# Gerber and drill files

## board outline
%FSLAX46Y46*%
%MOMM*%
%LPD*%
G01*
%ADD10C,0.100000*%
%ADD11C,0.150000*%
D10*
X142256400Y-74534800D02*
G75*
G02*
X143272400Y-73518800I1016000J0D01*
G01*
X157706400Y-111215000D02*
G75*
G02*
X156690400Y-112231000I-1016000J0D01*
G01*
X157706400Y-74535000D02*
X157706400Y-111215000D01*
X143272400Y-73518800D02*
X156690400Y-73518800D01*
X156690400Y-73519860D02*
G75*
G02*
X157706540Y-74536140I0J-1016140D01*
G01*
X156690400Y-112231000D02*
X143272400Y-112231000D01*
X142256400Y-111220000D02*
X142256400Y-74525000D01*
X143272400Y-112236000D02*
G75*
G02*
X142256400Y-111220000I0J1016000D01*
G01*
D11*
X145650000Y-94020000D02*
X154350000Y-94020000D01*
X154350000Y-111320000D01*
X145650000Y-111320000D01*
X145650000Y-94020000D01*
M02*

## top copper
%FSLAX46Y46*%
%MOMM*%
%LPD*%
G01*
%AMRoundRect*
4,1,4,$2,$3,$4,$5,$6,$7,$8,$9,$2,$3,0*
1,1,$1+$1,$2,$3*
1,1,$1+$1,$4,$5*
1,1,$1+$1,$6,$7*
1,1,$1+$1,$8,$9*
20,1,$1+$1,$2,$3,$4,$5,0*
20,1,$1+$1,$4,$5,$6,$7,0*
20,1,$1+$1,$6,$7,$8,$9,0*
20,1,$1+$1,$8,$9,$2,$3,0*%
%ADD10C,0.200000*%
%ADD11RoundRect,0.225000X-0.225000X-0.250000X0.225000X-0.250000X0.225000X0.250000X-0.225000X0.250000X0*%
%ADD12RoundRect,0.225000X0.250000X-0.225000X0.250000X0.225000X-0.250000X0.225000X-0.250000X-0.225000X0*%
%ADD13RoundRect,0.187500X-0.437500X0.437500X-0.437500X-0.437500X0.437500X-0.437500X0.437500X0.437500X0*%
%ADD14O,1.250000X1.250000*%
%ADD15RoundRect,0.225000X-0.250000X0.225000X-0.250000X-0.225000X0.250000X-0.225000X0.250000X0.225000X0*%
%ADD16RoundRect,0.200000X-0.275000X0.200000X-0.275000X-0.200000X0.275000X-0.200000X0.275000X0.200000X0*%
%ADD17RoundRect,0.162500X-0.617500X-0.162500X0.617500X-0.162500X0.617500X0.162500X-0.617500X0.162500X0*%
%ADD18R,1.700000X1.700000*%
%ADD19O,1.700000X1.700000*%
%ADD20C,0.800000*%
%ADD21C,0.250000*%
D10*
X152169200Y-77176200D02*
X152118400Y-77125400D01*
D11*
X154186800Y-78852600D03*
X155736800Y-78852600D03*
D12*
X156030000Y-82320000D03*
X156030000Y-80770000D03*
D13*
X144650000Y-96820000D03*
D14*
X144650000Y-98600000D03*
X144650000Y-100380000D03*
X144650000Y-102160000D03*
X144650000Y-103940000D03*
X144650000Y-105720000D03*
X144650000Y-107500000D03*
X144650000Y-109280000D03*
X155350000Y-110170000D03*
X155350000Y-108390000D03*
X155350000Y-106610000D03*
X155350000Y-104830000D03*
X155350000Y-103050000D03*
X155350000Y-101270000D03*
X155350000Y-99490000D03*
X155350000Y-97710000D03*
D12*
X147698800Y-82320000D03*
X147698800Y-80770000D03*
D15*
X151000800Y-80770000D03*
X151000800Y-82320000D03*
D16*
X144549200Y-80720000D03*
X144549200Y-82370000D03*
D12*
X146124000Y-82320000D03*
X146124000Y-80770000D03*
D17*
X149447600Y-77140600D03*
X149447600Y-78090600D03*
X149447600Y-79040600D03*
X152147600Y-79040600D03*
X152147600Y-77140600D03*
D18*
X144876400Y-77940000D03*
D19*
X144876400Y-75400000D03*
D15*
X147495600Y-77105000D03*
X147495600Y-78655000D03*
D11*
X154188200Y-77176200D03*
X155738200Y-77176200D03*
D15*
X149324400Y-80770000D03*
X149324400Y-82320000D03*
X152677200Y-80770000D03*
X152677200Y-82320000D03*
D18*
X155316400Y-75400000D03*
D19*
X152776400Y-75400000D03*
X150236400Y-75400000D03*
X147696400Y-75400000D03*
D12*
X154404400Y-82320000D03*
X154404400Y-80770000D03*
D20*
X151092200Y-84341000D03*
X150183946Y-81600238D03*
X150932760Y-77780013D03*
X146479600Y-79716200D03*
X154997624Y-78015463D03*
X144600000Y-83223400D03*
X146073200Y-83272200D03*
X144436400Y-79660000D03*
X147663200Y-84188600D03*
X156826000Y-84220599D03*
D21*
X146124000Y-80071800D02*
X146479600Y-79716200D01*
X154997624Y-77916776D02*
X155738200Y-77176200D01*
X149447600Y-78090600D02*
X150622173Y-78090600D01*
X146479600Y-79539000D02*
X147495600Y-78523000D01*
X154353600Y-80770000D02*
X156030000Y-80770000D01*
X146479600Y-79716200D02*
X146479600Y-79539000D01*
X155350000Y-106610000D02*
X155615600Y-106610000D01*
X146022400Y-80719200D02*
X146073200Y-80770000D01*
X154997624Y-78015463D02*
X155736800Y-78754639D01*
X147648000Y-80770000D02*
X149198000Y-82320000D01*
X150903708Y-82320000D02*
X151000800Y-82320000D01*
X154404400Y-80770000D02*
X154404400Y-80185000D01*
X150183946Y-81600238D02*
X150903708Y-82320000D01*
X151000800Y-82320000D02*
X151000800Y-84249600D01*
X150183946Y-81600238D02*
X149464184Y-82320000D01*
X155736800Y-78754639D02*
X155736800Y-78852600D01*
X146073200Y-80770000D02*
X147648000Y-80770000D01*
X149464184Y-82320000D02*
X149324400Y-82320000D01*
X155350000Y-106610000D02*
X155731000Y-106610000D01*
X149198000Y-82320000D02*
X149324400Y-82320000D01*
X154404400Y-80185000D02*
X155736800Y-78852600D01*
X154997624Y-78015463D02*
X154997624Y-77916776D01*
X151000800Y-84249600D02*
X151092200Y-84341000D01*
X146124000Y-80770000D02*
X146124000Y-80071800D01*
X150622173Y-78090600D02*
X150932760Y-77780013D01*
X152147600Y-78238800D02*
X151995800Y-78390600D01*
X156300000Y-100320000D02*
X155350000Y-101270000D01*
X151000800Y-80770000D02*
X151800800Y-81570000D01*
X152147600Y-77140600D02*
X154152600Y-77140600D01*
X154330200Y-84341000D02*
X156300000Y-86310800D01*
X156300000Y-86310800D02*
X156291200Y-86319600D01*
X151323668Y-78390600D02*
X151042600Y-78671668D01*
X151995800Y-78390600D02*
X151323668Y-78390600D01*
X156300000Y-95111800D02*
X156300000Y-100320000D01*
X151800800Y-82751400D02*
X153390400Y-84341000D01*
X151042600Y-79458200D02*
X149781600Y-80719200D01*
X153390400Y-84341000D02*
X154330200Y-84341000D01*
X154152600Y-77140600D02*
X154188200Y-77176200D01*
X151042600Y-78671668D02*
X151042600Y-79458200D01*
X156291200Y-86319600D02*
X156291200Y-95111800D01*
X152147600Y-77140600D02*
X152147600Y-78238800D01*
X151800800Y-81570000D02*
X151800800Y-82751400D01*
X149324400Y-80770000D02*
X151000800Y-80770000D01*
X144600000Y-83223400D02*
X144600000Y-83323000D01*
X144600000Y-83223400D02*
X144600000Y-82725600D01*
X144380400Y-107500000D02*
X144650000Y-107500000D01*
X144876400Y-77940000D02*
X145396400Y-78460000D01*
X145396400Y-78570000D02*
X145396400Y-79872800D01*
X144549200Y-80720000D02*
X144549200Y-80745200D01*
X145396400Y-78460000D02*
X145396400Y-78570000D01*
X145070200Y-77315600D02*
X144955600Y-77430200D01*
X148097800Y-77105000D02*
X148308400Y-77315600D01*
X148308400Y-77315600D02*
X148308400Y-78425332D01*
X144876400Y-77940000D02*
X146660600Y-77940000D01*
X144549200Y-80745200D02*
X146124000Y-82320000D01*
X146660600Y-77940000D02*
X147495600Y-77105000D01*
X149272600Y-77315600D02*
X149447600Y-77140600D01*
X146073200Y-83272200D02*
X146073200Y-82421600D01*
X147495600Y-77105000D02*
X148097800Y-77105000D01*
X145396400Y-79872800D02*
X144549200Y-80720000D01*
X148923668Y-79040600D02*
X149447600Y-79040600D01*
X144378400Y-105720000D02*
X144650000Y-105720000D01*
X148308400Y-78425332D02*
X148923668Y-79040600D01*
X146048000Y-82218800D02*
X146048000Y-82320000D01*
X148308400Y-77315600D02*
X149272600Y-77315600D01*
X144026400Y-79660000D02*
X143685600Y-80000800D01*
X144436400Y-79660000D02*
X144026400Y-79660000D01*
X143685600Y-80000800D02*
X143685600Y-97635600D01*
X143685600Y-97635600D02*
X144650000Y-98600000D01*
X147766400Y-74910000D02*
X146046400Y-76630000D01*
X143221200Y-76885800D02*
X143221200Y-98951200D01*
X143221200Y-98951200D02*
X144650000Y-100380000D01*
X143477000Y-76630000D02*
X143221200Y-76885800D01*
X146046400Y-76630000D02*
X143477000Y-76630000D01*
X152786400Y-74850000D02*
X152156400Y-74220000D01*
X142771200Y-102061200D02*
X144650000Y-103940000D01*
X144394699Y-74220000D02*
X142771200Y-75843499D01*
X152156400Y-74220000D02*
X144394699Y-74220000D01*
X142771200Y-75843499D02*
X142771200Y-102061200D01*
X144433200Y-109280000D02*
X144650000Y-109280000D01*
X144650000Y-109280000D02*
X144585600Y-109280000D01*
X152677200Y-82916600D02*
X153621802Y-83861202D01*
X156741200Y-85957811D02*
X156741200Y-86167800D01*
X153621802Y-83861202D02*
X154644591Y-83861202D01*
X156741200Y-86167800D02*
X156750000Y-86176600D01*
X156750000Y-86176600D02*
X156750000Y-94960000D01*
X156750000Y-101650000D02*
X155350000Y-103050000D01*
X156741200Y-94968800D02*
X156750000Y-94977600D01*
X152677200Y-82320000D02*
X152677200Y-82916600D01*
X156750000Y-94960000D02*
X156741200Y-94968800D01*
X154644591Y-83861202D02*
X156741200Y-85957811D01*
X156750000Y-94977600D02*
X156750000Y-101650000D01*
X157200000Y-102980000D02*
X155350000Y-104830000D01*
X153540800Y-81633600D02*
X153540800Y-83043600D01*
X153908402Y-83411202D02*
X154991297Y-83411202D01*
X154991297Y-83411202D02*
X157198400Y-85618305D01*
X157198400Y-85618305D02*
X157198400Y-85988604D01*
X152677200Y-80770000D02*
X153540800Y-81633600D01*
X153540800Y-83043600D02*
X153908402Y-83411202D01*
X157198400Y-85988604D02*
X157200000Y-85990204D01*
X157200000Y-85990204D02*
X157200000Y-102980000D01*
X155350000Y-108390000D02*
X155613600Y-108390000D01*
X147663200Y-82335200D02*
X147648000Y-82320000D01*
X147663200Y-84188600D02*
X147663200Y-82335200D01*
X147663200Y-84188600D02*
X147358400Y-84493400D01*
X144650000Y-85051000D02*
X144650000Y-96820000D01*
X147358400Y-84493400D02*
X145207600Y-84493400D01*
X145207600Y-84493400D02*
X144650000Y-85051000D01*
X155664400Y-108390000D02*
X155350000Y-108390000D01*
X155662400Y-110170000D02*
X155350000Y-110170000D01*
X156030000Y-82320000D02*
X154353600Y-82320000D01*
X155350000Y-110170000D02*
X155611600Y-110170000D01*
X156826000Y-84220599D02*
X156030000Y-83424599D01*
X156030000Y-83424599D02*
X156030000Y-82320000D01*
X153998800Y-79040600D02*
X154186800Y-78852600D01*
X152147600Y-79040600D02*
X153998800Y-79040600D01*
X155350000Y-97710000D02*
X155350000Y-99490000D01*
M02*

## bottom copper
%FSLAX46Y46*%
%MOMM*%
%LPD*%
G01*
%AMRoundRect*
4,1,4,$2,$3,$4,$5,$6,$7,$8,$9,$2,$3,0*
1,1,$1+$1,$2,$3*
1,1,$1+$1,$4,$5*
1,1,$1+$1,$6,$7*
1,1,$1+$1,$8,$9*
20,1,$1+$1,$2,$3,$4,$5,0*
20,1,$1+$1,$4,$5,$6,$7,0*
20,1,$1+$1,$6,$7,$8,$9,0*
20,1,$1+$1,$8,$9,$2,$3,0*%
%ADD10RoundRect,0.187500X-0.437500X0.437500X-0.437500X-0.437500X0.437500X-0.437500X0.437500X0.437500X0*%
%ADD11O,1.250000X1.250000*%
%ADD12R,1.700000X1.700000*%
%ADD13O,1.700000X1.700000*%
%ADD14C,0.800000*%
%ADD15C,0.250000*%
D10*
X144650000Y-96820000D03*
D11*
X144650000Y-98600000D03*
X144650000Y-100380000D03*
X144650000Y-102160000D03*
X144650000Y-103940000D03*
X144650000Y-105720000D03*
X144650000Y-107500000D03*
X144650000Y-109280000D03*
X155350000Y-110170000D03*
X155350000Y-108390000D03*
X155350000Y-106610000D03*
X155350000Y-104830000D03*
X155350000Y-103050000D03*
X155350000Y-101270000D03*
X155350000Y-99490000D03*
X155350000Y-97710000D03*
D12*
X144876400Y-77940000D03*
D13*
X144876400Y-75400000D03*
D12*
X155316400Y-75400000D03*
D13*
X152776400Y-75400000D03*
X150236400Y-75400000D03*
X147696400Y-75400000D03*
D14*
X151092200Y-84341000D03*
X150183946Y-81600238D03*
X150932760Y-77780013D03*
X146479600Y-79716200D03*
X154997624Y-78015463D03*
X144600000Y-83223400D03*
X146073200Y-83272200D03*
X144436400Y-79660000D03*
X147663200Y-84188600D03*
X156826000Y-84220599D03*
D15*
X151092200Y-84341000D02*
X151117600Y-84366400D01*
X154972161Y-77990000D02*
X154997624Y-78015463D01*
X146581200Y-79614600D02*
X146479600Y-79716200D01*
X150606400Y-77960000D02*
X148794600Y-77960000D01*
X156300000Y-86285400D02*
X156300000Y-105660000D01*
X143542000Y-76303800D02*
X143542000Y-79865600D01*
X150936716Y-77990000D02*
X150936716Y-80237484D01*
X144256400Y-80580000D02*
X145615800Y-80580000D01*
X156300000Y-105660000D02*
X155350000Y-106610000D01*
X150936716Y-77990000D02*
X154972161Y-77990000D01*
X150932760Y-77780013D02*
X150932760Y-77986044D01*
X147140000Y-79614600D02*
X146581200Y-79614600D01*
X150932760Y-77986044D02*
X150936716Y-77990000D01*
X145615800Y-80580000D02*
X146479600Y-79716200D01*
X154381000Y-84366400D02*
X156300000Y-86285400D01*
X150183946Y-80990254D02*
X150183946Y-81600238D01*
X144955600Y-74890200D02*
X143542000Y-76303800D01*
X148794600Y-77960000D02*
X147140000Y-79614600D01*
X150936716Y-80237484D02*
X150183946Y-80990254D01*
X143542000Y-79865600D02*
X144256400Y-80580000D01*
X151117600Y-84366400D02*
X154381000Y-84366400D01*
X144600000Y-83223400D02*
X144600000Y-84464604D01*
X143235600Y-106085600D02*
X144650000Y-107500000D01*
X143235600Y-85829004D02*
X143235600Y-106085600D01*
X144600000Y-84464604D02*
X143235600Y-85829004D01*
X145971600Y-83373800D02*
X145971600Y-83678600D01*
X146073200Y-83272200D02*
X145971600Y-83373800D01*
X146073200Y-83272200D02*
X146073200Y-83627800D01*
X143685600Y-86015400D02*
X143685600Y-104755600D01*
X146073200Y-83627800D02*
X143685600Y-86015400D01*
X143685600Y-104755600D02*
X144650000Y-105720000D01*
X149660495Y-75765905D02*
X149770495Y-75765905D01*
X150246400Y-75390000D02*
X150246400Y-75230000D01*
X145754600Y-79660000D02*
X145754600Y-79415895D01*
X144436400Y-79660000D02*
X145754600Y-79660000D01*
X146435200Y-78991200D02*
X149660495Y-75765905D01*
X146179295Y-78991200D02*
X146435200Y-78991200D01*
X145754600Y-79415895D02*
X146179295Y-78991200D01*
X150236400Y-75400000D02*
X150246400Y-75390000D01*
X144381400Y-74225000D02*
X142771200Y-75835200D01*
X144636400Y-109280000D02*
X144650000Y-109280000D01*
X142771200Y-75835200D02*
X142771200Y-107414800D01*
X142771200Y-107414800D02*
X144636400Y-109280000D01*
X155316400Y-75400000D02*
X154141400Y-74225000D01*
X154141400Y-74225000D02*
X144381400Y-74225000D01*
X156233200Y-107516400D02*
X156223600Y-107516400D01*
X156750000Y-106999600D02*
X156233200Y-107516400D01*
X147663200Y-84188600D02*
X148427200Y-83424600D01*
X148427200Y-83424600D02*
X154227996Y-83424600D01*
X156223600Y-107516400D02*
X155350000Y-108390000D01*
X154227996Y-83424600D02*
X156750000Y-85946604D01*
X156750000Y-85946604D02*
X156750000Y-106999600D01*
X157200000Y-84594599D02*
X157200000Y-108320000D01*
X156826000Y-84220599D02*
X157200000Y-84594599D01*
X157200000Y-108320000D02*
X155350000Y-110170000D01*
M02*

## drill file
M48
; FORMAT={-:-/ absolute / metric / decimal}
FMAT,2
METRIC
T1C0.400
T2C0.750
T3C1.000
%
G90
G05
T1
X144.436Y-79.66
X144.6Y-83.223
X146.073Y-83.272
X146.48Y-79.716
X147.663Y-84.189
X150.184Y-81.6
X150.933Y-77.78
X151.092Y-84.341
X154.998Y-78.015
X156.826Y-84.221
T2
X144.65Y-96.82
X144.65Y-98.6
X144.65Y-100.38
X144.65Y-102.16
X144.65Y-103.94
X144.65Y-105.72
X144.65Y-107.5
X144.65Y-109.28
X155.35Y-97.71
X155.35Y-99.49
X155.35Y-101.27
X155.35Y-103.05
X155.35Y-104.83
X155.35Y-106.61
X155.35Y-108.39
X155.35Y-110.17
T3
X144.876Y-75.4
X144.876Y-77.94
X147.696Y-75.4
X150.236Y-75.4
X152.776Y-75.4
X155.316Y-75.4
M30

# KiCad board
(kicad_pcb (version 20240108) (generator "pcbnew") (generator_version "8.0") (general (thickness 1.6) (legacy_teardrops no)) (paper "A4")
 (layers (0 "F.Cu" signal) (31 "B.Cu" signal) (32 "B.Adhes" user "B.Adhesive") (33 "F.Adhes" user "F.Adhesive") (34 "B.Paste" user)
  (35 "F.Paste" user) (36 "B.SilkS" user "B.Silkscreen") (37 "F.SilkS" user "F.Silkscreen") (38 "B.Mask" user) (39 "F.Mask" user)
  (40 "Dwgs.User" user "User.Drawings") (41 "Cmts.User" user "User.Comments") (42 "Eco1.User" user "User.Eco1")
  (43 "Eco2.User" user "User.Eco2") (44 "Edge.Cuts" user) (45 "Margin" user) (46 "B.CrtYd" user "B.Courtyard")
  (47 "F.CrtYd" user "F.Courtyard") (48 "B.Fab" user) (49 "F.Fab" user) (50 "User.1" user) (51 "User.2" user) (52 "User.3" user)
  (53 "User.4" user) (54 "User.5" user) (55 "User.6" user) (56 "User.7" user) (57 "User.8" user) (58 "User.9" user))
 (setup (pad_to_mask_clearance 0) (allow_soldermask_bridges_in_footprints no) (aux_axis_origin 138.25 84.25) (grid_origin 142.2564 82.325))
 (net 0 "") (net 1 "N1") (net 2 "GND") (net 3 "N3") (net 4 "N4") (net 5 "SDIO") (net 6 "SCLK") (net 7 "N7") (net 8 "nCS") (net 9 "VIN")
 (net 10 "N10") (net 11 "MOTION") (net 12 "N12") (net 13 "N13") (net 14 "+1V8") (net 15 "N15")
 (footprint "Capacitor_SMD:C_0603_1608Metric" (layer "F.Cu") (at 154.9618 78.8526)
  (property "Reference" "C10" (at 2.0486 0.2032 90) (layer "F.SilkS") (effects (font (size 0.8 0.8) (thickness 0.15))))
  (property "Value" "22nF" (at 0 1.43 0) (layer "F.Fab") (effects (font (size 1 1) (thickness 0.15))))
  (pad "1" smd roundrect (at -0.775 0) (size 0.9 0.95) (layers "F.Cu" "F.Paste" "F.Mask") (roundrect_rratio 0.25) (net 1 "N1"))
  (pad "2" smd roundrect (at 0.775 0) (size 0.9 0.95) (layers "F.Cu" "F.Paste" "F.Mask") (roundrect_rratio 0.25) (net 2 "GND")))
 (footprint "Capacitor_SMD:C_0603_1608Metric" (layer "F.Cu") (at 156.03 81.545 90)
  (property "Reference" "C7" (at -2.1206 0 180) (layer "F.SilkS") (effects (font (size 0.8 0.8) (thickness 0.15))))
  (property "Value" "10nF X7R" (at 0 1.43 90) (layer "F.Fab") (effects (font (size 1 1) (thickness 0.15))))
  (pad "1" smd roundrect (at -0.775 0 90) (size 0.9 0.95) (layers "F.Cu" "F.Paste" "F.Mask") (roundrect_rratio 0.25) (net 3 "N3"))
  (pad "2" smd roundrect (at 0.775 0 90) (size 0.9 0.95) (layers "F.Cu" "F.Paste" "F.Mask") (roundrect_rratio 0.25) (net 2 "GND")))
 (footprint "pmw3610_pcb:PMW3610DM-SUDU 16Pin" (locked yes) (layer "F.Cu") (at 150 102.988 90)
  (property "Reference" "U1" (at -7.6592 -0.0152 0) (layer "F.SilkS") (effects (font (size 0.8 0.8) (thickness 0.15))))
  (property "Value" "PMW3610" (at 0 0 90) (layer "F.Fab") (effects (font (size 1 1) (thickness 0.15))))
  (fp_rect (start 8.968 -4.35) (end -8.332 4.35) (stroke (width 0.15) (type solid)) (fill none) (layer "Edge.Cuts"))
  (pad "1" thru_hole roundrect (at 6.168 -5.35 270) (size 1.25 1.25) (drill 0.75) (layers "*.Cu" "*.Mask") (remove_unused_layers no)
   (roundrect_rratio 0.15) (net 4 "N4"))
  (pad "2" thru_hole oval (at 4.388 -5.35 270) (size 1.25 1.25) (drill 0.75) (layers "*.Cu" "*.Mask") (remove_unused_layers no)
   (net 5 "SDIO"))
  (pad "3" thru_hole oval (at 2.608 -5.35 270) (size 1.25 1.25) (drill 0.75) (layers "*.Cu" "*.Mask") (remove_unused_layers no)
   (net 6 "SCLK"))
  (pad "4" thru_hole oval (at 0.828 -5.35 270) (size 1.25 1.25) (drill 0.75) (layers "*.Cu" "*.Mask") (remove_unused_layers no) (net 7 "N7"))
  (pad "5" thru_hole oval (at -0.952 -5.35 270) (size 1.25 1.25) (drill 0.75) (layers "*.Cu" "*.Mask") (remove_unused_layers no)
   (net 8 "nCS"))
  (pad "6" thru_hole oval (at -2.732 -5.35 270) (size 1.25 1.25) (drill 0.75) (layers "*.Cu" "*.Mask") (remove_unused_layers no)
   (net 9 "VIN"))
  (pad "7" thru_hole oval (at -4.512 -5.35 270) (size 1.25 1.25) (drill 0.75) (layers "*.Cu" "*.Mask") (remove_unused_layers no)
   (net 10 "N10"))
  (pad "8" thru_hole oval (at -6.292 -5.35 270) (size 1.25 1.25) (drill 0.75) (layers "*.Cu" "*.Mask") (remove_unused_layers no)
   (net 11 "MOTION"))
  (pad "9" thru_hole oval (at -7.182 5.35 270) (size 1.25 1.25) (drill 0.75) (layers "*.Cu" "*.Mask") (remove_unused_layers no) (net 3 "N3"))
  (pad "10" thru_hole oval (at -5.402 5.35 270) (size 1.25 1.25) (drill 0.75) (layers "*.Cu" "*.Mask") (remove_unused_layers no)
   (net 4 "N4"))
  (pad "11" thru_hole oval (at -3.622 5.35 270) (size 1.25 1.25) (drill 0.75) (layers "*.Cu" "*.Mask") (remove_unused_layers no)
   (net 2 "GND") (thermal_bridge_angle 45))
  (pad "12" thru_hole oval (at -1.842 5.35 270) (size 1.25 1.25) (drill 0.75) (layers "*.Cu" "*.Mask") (remove_unused_layers no)
   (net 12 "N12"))
  (pad "13" thru_hole oval (at -0.062 5.35 270) (size 1.25 1.25) (drill 0.75) (layers "*.Cu" "*.Mask") (remove_unused_layers no)
   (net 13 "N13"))
  (pad "14" thru_hole oval (at 1.718 5.35 270) (size 1.25 1.25) (drill 0.75) (layers "*.Cu" "*.Mask") (remove_unused_layers no)
   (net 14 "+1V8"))
  (pad "15" thru_hole oval (at 3.498 5.35 270) (size 1.25 1.25) (drill 0.75) (layers "*.Cu" "*.Mask") (remove_unused_layers no)
   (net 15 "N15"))
  (pad "16" thru_hole oval (at 5.278 5.35 270) (size 1.25 1.25) (drill 0.75) (layers "*.Cu" "*.Mask") (remove_unused_layers no)
   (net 15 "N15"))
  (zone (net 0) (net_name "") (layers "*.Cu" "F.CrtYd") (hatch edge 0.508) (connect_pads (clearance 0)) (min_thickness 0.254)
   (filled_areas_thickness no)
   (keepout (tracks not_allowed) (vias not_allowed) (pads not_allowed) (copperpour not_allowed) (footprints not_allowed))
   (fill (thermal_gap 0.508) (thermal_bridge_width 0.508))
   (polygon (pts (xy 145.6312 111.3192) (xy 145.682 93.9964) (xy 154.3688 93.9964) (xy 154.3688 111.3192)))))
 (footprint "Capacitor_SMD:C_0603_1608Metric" (layer "F.Cu") (at 147.6988 81.545 90)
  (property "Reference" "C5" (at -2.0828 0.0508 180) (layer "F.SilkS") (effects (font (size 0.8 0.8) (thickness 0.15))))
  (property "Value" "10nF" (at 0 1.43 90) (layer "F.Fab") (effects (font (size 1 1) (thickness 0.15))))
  (pad "1" smd roundrect (at -0.775 0 90) (size 0.9 0.95) (layers "F.Cu" "F.Paste" "F.Mask") (roundrect_rratio 0.25) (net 4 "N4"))
  (pad "2" smd roundrect (at 0.775 0 90) (size 0.9 0.95) (layers "F.Cu" "F.Paste" "F.Mask") (roundrect_rratio 0.25) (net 2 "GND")))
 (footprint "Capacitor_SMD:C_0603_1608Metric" (layer "F.Cu") (at 151.0008 81.545 -90)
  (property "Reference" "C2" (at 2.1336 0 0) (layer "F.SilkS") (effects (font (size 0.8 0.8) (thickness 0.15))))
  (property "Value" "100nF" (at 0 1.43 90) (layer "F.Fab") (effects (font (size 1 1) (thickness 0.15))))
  (pad "1" smd roundrect (at -0.775 0 270) (size 0.9 0.95) (layers "F.Cu" "F.Paste" "F.Mask") (roundrect_rratio 0.25) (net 14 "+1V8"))
  (pad "2" smd roundrect (at 0.775 0 270) (size 0.9 0.95) (layers "F.Cu" "F.Paste" "F.Mask") (roundrect_rratio 0.25) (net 2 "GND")))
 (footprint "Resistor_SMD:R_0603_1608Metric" (layer "F.Cu") (at 144.5492 81.545 -90)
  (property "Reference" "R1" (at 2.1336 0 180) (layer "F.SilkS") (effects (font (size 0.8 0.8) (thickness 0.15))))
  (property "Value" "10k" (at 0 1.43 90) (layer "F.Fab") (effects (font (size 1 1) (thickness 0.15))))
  (pad "1" smd roundrect (at -0.825 0 270) (size 0.8 0.95) (layers "F.Cu" "F.Paste" "F.Mask") (roundrect_rratio 0.25) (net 9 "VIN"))
  (pad "2" smd roundrect (at 0.825 0 270) (size 0.8 0.95) (layers "F.Cu" "F.Paste" "F.Mask") (roundrect_rratio 0.25) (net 10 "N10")))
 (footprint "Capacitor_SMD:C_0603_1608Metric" (layer "F.Cu") (at 146.124 81.545 90)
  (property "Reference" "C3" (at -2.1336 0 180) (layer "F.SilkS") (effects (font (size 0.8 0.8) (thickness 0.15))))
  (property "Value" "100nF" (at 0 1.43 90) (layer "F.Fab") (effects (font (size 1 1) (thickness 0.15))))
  (pad "1" smd roundrect (at -0.775 0 90) (size 0.9 0.95) (layers "F.Cu" "F.Paste" "F.Mask") (roundrect_rratio 0.25) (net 9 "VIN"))
  (pad "2" smd roundrect (at 0.775 0 90) (size 0.9 0.95) (layers "F.Cu" "F.Paste" "F.Mask") (roundrect_rratio 0.25) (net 2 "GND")))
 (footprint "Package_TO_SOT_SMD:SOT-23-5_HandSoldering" (layer "F.Cu") (at 150.7976 78.0906)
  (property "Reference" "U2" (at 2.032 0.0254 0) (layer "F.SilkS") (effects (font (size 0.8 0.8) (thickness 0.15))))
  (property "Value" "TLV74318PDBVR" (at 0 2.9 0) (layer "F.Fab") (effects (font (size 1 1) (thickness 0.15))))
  (pad "1" smd roundrect (at -1.35 -0.95) (size 1.56 0.65) (layers "F.Cu" "F.Paste" "F.Mask") (roundrect_rratio 0.25) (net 9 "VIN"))
  (pad "2" smd roundrect (at -1.35 0) (size 1.56 0.65) (layers "F.Cu" "F.Paste" "F.Mask") (roundrect_rratio 0.25) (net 2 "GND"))
  (pad "3" smd roundrect (at -1.35 0.95) (size 1.56 0.65) (layers "F.Cu" "F.Paste" "F.Mask") (roundrect_rratio 0.25) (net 9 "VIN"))
  (pad "4" smd roundrect (at 1.35 0.95) (size 1.56 0.65) (layers "F.Cu" "F.Paste" "F.Mask") (roundrect_rratio 0.25) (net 1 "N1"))
  (pad "5" smd roundrect (at 1.35 -0.95) (size 1.56 0.65) (layers "F.Cu" "F.Paste" "F.Mask") (roundrect_rratio 0.25) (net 14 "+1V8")))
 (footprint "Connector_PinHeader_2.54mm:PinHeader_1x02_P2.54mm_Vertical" (layer "F.Cu") (at 144.8764 77.94 180)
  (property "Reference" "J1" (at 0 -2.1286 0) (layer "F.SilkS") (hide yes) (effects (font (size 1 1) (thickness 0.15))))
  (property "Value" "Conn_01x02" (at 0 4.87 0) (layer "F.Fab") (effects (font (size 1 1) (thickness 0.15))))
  (pad "1" thru_hole rect (at 0 0 180) (size 1.7 1.7) (drill 1) (layers "*.Cu" "*.Mask") (remove_unused_layers no) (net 9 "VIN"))
  (pad "2" thru_hole oval (at 0 2.54 180) (size 1.7 1.7) (drill 1) (layers "*.Cu" "*.Mask") (remove_unused_layers no) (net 2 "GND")))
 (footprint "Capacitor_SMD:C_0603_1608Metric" (layer "F.Cu") (at 147.4956 77.88 -90)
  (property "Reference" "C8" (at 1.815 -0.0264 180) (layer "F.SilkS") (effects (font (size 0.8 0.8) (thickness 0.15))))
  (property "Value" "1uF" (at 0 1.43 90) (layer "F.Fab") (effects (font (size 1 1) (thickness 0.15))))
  (pad "1" smd roundrect (at -0.775 0 270) (size 0.9 0.95) (layers "F.Cu" "F.Paste" "F.Mask") (roundrect_rratio 0.25) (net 9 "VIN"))
  (pad "2" smd roundrect (at 0.775 0 270) (size 0.9 0.95) (layers "F.Cu" "F.Paste" "F.Mask") (roundrect_rratio 0.25) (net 2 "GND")))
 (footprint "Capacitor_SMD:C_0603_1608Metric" (layer "F.Cu") (at 154.9632 77.1762)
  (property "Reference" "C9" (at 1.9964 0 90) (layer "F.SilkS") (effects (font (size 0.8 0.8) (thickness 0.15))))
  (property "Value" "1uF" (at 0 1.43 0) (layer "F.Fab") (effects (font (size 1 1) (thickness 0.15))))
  (pad "1" smd roundrect (at -0.775 0) (size 0.9 0.95) (layers "F.Cu" "F.Paste" "F.Mask") (roundrect_rratio 0.25) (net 14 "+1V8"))
  (pad "2" smd roundrect (at 0.775 0) (size 0.9 0.95) (layers "F.Cu" "F.Paste" "F.Mask") (roundrect_rratio 0.25) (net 2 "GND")))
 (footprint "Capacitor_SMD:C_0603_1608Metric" (layer "F.Cu") (at 149.3244 81.545 -90)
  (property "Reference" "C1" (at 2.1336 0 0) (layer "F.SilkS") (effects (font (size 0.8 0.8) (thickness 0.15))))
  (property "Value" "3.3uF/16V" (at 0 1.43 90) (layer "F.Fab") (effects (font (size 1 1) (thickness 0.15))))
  (pad "1" smd roundrect (at -0.775 0 270) (size 0.9 0.95) (layers "F.Cu" "F.Paste" "F.Mask") (roundrect_rratio 0.25) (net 14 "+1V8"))
  (pad "2" smd roundrect (at 0.775 0 270) (size 0.9 0.95) (layers "F.Cu" "F.Paste" "F.Mask") (roundrect_rratio 0.25) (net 2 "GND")))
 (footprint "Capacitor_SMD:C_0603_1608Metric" (layer "F.Cu") (at 152.6772 81.545 -90)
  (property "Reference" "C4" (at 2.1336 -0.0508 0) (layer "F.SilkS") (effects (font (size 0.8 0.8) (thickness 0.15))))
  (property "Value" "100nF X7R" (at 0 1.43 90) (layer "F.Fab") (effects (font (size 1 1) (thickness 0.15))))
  (pad "1" smd roundrect (at -0.775 0 270) (size 0.9 0.95) (layers "F.Cu" "F.Paste" "F.Mask") (roundrect_rratio 0.25) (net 12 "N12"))
  (pad "2" smd roundrect (at 0.775 0 270) (size 0.9 0.95) (layers "F.Cu" "F.Paste" "F.Mask") (roundrect_rratio 0.25) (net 13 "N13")))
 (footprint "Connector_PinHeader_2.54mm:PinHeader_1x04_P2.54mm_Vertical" (layer "F.Cu") (at 155.3164 75.4 -90)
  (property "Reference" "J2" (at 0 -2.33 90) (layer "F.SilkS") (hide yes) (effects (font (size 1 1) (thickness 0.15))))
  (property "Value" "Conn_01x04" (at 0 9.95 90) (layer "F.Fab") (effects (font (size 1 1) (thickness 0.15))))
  (pad "1" thru_hole rect (at 0 0 270) (size 1.7 1.7) (drill 1) (layers "*.Cu" "*.Mask") (remove_unused_layers no) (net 11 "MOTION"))
  (pad "2" thru_hole oval (at 0 2.54 270) (size 1.7 1.7) (drill 1) (layers "*.Cu" "*.Mask") (remove_unused_layers no) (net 8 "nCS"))
  (pad "3" thru_hole oval (at 0 5.08 270) (size 1.7 1.7) (drill 1) (layers "*.Cu" "*.Mask") (remove_unused_layers no) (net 5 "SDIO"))
  (pad "4" thru_hole oval (at 0 7.62 270) (size 1.7 1.7) (drill 1) (layers "*.Cu" "*.Mask") (remove_unused_layers no) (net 6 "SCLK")))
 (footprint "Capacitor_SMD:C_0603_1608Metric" (layer "F.Cu") (at 154.4044 81.545 90)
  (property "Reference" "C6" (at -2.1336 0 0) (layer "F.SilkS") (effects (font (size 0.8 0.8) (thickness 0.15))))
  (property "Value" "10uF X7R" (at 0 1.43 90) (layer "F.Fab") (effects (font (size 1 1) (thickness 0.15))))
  (pad "1" smd roundrect (at -0.775 0 90) (size 0.9 0.95) (layers "F.Cu" "F.Paste" "F.Mask") (roundrect_rratio 0.25) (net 3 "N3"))
  (pad "2" smd roundrect (at 0.775 0 90) (size 0.9 0.95) (layers "F.Cu" "F.Paste" "F.Mask") (roundrect_rratio 0.25) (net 2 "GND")))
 (gr_line (start 152.1692 77.1762) (end 152.1184 77.1254) (stroke (width 0.2) (type default)) (layer "F.Cu") (net 14))
 (gr_arc (start 142.2564 74.5348) (mid 142.55398 73.81638) (end 143.2724 73.5188) (stroke (width 0.1) (type default)) (layer "Edge.Cuts"))
 (gr_arc (start 157.7064 111.215) (mid 157.40882 111.93342) (end 156.6904 112.231) (stroke (width 0.1) (type default)) (layer "Edge.Cuts"))
 (gr_line (start 157.7064 74.535) (end 157.7064 111.215) (stroke (width 0.1) (type default)) (layer "Edge.Cuts"))
 (gr_line (start 143.2724 73.5188) (end 156.6904 73.5188) (stroke (width 0.1) (type default)) (layer "Edge.Cuts"))
 (gr_arc (start 156.6904 73.51986) (mid 157.408969 73.81753) (end 157.70654 74.53614) (stroke (width 0.1) (type default))
  (layer "Edge.Cuts"))
 (gr_line (start 156.6904 112.231) (end 143.2724 112.231) (stroke (width 0.1) (type default)) (layer "Edge.Cuts"))
 (gr_line (start 142.2564 111.22) (end 142.2564 74.525) (stroke (width 0.1) (type default)) (layer "Edge.Cuts"))
 (gr_arc (start 143.2724 112.236) (mid 142.55398 111.93842) (end 142.2564 111.22) (stroke (width 0.1) (type default)) (layer "Edge.Cuts"))
 (segment (start 146.124 80.0718) (end 146.4796 79.7162) (width 0.25) (layer "F.Cu") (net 2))
 (segment (start 154.997624 77.916776) (end 155.7382 77.1762) (width 0.25) (layer "F.Cu") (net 2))
 (segment (start 149.4476 78.0906) (end 150.622173 78.0906) (width 0.25) (layer "F.Cu") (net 2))
 (segment (start 146.4796 79.539) (end 147.4956 78.523) (width 0.25) (layer "F.Cu") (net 2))
 (segment (start 154.3536 80.77) (end 156.03 80.77) (width 0.25) (layer "F.Cu") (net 2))
 (segment (start 146.4796 79.7162) (end 146.4796 79.539) (width 0.25) (layer "F.Cu") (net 2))
 (segment (start 155.35 106.61) (end 155.6156 106.61) (width 0.25) (layer "F.Cu") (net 2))
 (segment (start 146.0224 80.7192) (end 146.0732 80.77) (width 0.25) (layer "F.Cu") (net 2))
 (segment (start 154.997624 78.015463) (end 155.7368 78.754639) (width 0.25) (layer "F.Cu") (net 2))
 (segment (start 147.648 80.77) (end 149.198 82.32) (width 0.25) (layer "F.Cu") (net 2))
 (segment (start 150.903708 82.32) (end 151.0008 82.32) (width 0.25) (layer "F.Cu") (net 2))
 (segment (start 154.4044 80.77) (end 154.4044 80.185) (width 0.25) (layer "F.Cu") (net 2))
 (segment (start 150.183946 81.600238) (end 150.903708 82.32) (width 0.25) (layer "F.Cu") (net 2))
 (segment (start 151.0008 82.32) (end 151.0008 84.2496) (width 0.25) (layer "F.Cu") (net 2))
 (segment (start 150.183946 81.600238) (end 149.464184 82.32) (width 0.25) (layer "F.Cu") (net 2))
 (segment (start 155.7368 78.754639) (end 155.7368 78.8526) (width 0.25) (layer "F.Cu") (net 2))
 (segment (start 146.0732 80.77) (end 147.648 80.77) (width 0.25) (layer "F.Cu") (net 2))
 (segment (start 149.464184 82.32) (end 149.3244 82.32) (width 0.25) (layer "F.Cu") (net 2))
 (segment (start 155.35 106.61) (end 155.731 106.61) (width 0.25) (layer "F.Cu") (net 2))
 (segment (start 149.198 82.32) (end 149.3244 82.32) (width 0.25) (layer "F.Cu") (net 2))
 (segment (start 154.4044 80.185) (end 155.7368 78.8526) (width 0.25) (layer "F.Cu") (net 2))
 (segment (start 154.997624 78.015463) (end 154.997624 77.916776) (width 0.25) (layer "F.Cu") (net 2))
 (segment (start 151.0008 84.2496) (end 151.0922 84.341) (width 0.25) (layer "F.Cu") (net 2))
 (segment (start 146.124 80.77) (end 146.124 80.0718) (width 0.25) (layer "F.Cu") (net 2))
 (segment (start 150.622173 78.0906) (end 150.93276 77.780013) (width 0.25) (layer "F.Cu") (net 2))
 (via (at 151.0922 84.341) (size 0.8) (drill 0.4) (layers "F.Cu" "B.Cu") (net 2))
 (via (at 150.183946 81.600238) (size 0.8) (drill 0.4) (layers "F.Cu" "B.Cu") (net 2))
 (via (at 150.93276 77.780013) (size 0.8) (drill 0.4) (layers "F.Cu" "B.Cu") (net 2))
 (via (at 146.4796 79.7162) (size 0.8) (drill 0.4) (layers "F.Cu" "B.Cu") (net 2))
 (via (at 154.997624 78.015463) (size 0.8) (drill 0.4) (layers "F.Cu" "B.Cu") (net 2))
 (segment (start 151.0922 84.341) (end 151.1176 84.3664) (width 0.25) (layer "B.Cu") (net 2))
 (segment (start 154.972161 77.99) (end 154.997624 78.015463) (width 0.25) (layer "B.Cu") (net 2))
 (segment (start 146.5812 79.6146) (end 146.4796 79.7162) (width 0.25) (layer "B.Cu") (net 2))
 (segment (start 150.6064 77.96) (end 148.7946 77.96) (width 0.25) (layer "B.Cu") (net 2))
 (segment (start 156.3 86.2854) (end 156.3 105.66) (width 0.25) (layer "B.Cu") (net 2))
 (segment (start 143.542 76.3038) (end 143.542 79.8656) (width 0.25) (layer "B.Cu") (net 2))
 (segment (start 150.936716 77.99) (end 150.936716 80.237484) (width 0.25) (layer "B.Cu") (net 2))
 (segment (start 144.2564 80.58) (end 145.6158 80.58) (width 0.25) (layer "B.Cu") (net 2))
 (segment (start 156.3 105.66) (end 155.35 106.61) (width 0.25) (layer "B.Cu") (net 2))
 (segment (start 150.936716 77.99) (end 154.972161 77.99) (width 0.25) (layer "B.Cu") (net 2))
 (segment (start 150.93276 77.780013) (end 150.93276 77.986044) (width 0.25) (layer "B.Cu") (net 2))
 (segment (start 147.14 79.6146) (end 146.5812 79.6146) (width 0.25) (layer "B.Cu") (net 2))
 (segment (start 150.93276 77.986044) (end 150.936716 77.99) (width 0.25) (layer "B.Cu") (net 2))
 (segment (start 145.6158 80.58) (end 146.4796 79.7162) (width 0.25) (layer "B.Cu") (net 2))
 (segment (start 154.381 84.3664) (end 156.3 86.2854) (width 0.25) (layer "B.Cu") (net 2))
 (segment (start 150.183946 80.990254) (end 150.183946 81.600238) (width 0.25) (layer "B.Cu") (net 2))
 (segment (start 144.9556 74.8902) (end 143.542 76.3038) (width 0.25) (layer "B.Cu") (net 2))
 (segment (start 148.7946 77.96) (end 147.14 79.6146) (width 0.25) (layer "B.Cu") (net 2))
 (segment (start 150.936716 80.237484) (end 150.183946 80.990254) (width 0.25) (layer "B.Cu") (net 2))
 (segment (start 143.542 79.8656) (end 144.2564 80.58) (width 0.25) (layer "B.Cu") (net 2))
 (segment (start 151.1176 84.3664) (end 154.381 84.3664) (width 0.25) (layer "B.Cu") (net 2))
 (segment (start 152.1476 78.2388) (end 151.9958 78.3906) (width 0.25) (layer "F.Cu") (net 14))
 (segment (start 156.3 100.32) (end 155.35 101.27) (width 0.25) (layer "F.Cu") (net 14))
 (segment (start 151.0008 80.77) (end 151.8008 81.57) (width 0.25) (layer "F.Cu") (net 14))
 (segment (start 152.1476 77.1406) (end 154.1526 77.1406) (width 0.25) (layer "F.Cu") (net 14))
 (segment (start 154.3302 84.341) (end 156.3 86.3108) (width 0.25) (layer "F.Cu") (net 14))
 (segment (start 156.3 86.3108) (end 156.2912 86.3196) (width 0.25) (layer "F.Cu") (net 14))
 (segment (start 151.323668 78.3906) (end 151.0426 78.671668) (width 0.25) (layer "F.Cu") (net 14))
 (segment (start 151.9958 78.3906) (end 151.323668 78.3906) (width 0.25) (layer "F.Cu") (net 14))
 (segment (start 156.3 95.1118) (end 156.3 100.32) (width 0.25) (layer "F.Cu") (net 14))
 (segment (start 151.8008 82.7514) (end 153.3904 84.341) (width 0.25) (layer "F.Cu") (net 14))
 (segment (start 151.0426 79.4582) (end 149.7816 80.7192) (width 0.25) (layer "F.Cu") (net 14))
 (segment (start 153.3904 84.341) (end 154.3302 84.341) (width 0.25) (layer "F.Cu") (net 14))
 (segment (start 154.1526 77.1406) (end 154.1882 77.1762) (width 0.25) (layer "F.Cu") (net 14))
 (segment (start 151.0426 78.671668) (end 151.0426 79.4582) (width 0.25) (layer "F.Cu") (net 14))
 (segment (start 156.2912 86.3196) (end 156.2912 95.1118) (width 0.25) (layer "F.Cu") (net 14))
 (segment (start 152.1476 77.1406) (end 152.1476 78.2388) (width 0.25) (layer "F.Cu") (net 14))
 (segment (start 151.8008 81.57) (end 151.8008 82.7514) (width 0.25) (layer "F.Cu") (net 14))
 (segment (start 149.3244 80.77) (end 151.0008 80.77) (width 0.25) (layer "F.Cu") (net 14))
 (segment (start 144.6 83.2234) (end 144.6 83.323) (width 0.25) (layer "F.Cu") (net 10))
 (segment (start 144.6 83.2234) (end 144.6 82.7256) (width 0.25) (layer "F.Cu") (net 10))
 (segment (start 144.3804 107.5) (end 144.65 107.5) (width 0.25) (layer "F.Cu") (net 10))
 (via (at 144.6 83.2234) (size 0.8) (drill 0.4) (layers "F.Cu" "B.Cu") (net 10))
 (segment (start 144.6 83.2234) (end 144.6 84.464604) (width 0.25) (layer "B.Cu") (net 10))
 (segment (start 143.2356 106.0856) (end 144.65 107.5) (width 0.25) (layer "B.Cu") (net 10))
 (segment (start 143.2356 85.829004) (end 143.2356 106.0856) (width 0.25) (layer "B.Cu") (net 10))
 (segment (start 144.6 84.464604) (end 143.2356 85.829004) (width 0.25) (layer "B.Cu") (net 10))
 (segment (start 144.8764 77.94) (end 145.3964 78.46) (width 0.25) (layer "F.Cu") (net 9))
 (segment (start 145.3964 78.57) (end 145.3964 79.8728) (width 0.25) (layer "F.Cu") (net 9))
 (segment (start 144.5492 80.72) (end 144.5492 80.7452) (width 0.25) (layer "F.Cu") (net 9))
 (segment (start 145.3964 78.46) (end 145.3964 78.57) (width 0.25) (layer "F.Cu") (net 9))
 (segment (start 145.0702 77.3156) (end 144.9556 77.4302) (width 0.25) (layer "F.Cu") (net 9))
 (segment (start 148.0978 77.105) (end 148.3084 77.3156) (width 0.25) (layer "F.Cu") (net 9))
 (segment (start 148.3084 77.3156) (end 148.3084 78.425332) (width 0.25) (layer "F.Cu") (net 9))
 (segment (start 144.8764 77.94) (end 146.6606 77.94) (width 0.25) (layer "F.Cu") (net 9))
 (segment (start 144.5492 80.7452) (end 146.124 82.32) (width 0.25) (layer "F.Cu") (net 9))
 (segment (start 146.6606 77.94) (end 147.4956 77.105) (width 0.25) (layer "F.Cu") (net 9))
 (segment (start 149.2726 77.3156) (end 149.4476 77.1406) (width 0.25) (layer "F.Cu") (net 9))
 (segment (start 146.0732 83.2722) (end 146.0732 82.4216) (width 0.25) (layer "F.Cu") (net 9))
 (segment (start 147.4956 77.105) (end 148.0978 77.105) (width 0.25) (layer "F.Cu") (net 9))
 (segment (start 145.3964 79.8728) (end 144.5492 80.72) (width 0.25) (layer "F.Cu") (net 9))
 (segment (start 148.923668 79.0406) (end 149.4476 79.0406) (width 0.25) (layer "F.Cu") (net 9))
 (segment (start 144.3784 105.72) (end 144.65 105.72) (width 0.25) (layer "F.Cu") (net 9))
 (segment (start 148.3084 78.425332) (end 148.923668 79.0406) (width 0.25) (layer "F.Cu") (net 9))
 (segment (start 146.048 82.2188) (end 146.048 82.32) (width 0.25) (layer "F.Cu") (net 9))
 (segment (start 148.3084 77.3156) (end 149.2726 77.3156) (width 0.25) (layer "F.Cu") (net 9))
 (via (at 146.0732 83.2722) (size 0.8) (drill 0.4) (layers "F.Cu" "B.Cu") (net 9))
 (segment (start 145.9716 83.3738) (end 145.9716 83.6786) (width 0.25) (layer "B.Cu") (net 9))
 (segment (start 146.0732 83.2722) (end 145.9716 83.3738) (width 0.25) (layer "B.Cu") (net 9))
 (segment (start 146.0732 83.2722) (end 146.0732 83.6278) (width 0.25) (layer "B.Cu") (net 9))
 (segment (start 143.6856 86.0154) (end 143.6856 104.7556) (width 0.25) (layer "B.Cu") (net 9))
 (segment (start 146.0732 83.6278) (end 143.6856 86.0154) (width 0.25) (layer "B.Cu") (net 9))
 (segment (start 143.6856 104.7556) (end 144.65 105.72) (width 0.25) (layer "B.Cu") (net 9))
 (segment (start 144.0264 79.66) (end 143.6856 80.0008) (width 0.25) (layer "F.Cu") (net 5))
 (segment (start 144.4364 79.66) (end 144.0264 79.66) (width 0.25) (layer "F.Cu") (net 5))
 (segment (start 143.6856 80.0008) (end 143.6856 97.6356) (width 0.25) (layer "F.Cu") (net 5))
 (segment (start 143.6856 97.6356) (end 144.65 98.6) (width 0.25) (layer "F.Cu") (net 5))
 (via (at 144.4364 79.66) (size 0.8) (drill 0.4) (layers "F.Cu" "B.Cu") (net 5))
 (segment (start 149.660495 75.765905) (end 149.770495 75.765905) (width 0.25) (layer "B.Cu") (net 5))
 (segment (start 150.2464 75.39) (end 150.2464 75.23) (width 0.25) (layer "B.Cu") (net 5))
 (segment (start 145.7546 79.66) (end 145.7546 79.415895) (width 0.25) (layer "B.Cu") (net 5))
 (segment (start 144.4364 79.66) (end 145.7546 79.66) (width 0.25) (layer "B.Cu") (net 5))
 (segment (start 146.4352 78.9912) (end 149.660495 75.765905) (width 0.25) (layer "B.Cu") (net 5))
 (segment (start 146.179295 78.9912) (end 146.4352 78.9912) (width 0.25) (layer "B.Cu") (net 5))
 (segment (start 145.7546 79.415895) (end 146.179295 78.9912) (width 0.25) (layer "B.Cu") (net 5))
 (segment (start 150.2364 75.4) (end 150.2464 75.39) (width 0.25) (layer "B.Cu") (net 5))
 (segment (start 147.7664 74.91) (end 146.0464 76.63) (width 0.25) (layer "F.Cu") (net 6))
 (segment (start 143.2212 76.8858) (end 143.2212 98.9512) (width 0.25) (layer "F.Cu") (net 6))
 (segment (start 143.2212 98.9512) (end 144.65 100.38) (width 0.25) (layer "F.Cu") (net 6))
 (segment (start 143.477 76.63) (end 143.2212 76.8858) (width 0.25) (layer "F.Cu") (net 6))
 (segment (start 146.0464 76.63) (end 143.477 76.63) (width 0.25) (layer "F.Cu") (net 6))
 (segment (start 152.7864 74.85) (end 152.1564 74.22) (width 0.25) (layer "F.Cu") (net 8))
 (segment (start 142.7712 102.0612) (end 144.65 103.94) (width 0.25) (layer "F.Cu") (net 8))
 (segment (start 144.394699 74.22) (end 142.7712 75.843499) (width 0.25) (layer "F.Cu") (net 8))
 (segment (start 152.1564 74.22) (end 144.394699 74.22) (width 0.25) (layer "F.Cu") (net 8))
 (segment (start 142.7712 75.843499) (end 142.7712 102.0612) (width 0.25) (layer "F.Cu") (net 8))
 (segment (start 144.4332 109.28) (end 144.65 109.28) (width 0.25) (layer "F.Cu") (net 11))
 (segment (start 144.65 109.28) (end 144.5856 109.28) (width 0.25) (layer "F.Cu") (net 11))
 (segment (start 144.3814 74.225) (end 142.7712 75.8352) (width 0.25) (layer "B.Cu") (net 11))
 (segment (start 144.6364 109.28) (end 144.65 109.28) (width 0.25) (layer "B.Cu") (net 11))
 (segment (start 142.7712 75.8352) (end 142.7712 107.4148) (width 0.25) (layer "B.Cu") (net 11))
 (segment (start 142.7712 107.4148) (end 144.6364 109.28) (width 0.25) (layer "B.Cu") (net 11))
 (segment (start 155.3164 75.4) (end 154.1414 74.225) (width 0.25) (layer "B.Cu") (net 11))
 (segment (start 154.1414 74.225) (end 144.3814 74.225) (width 0.25) (layer "B.Cu") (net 11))
 (segment (start 152.6772 82.9166) (end 153.621802 83.861202) (width 0.25) (layer "F.Cu") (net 13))
 (segment (start 156.7412 85.957811) (end 156.7412 86.1678) (width 0.25) (layer "F.Cu") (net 13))
 (segment (start 153.621802 83.861202) (end 154.644591 83.861202) (width 0.25) (layer "F.Cu") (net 13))
 (segment (start 156.7412 86.1678) (end 156.75 86.1766) (width 0.25) (layer "F.Cu") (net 13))
 (segment (start 156.75 86.1766) (end 156.75 94.96) (width 0.25) (layer "F.Cu") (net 13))
 (segment (start 156.75 101.65) (end 155.35 103.05) (width 0.25) (layer "F.Cu") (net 13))
 (segment (start 156.7412 94.9688) (end 156.75 94.9776) (width 0.25) (layer "F.Cu") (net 13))
 (segment (start 152.6772 82.32) (end 152.6772 82.9166) (width 0.25) (layer "F.Cu") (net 13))
 (segment (start 156.75 94.96) (end 156.7412 94.9688) (width 0.25) (layer "F.Cu") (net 13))
 (segment (start 154.644591 83.861202) (end 156.7412 85.957811) (width 0.25) (layer "F.Cu") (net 13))
 (segment (start 156.75 94.9776) (end 156.75 101.65) (width 0.25) (layer "F.Cu") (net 13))
 (segment (start 157.2 102.98) (end 155.35 104.83) (width 0.25) (layer "F.Cu") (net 12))
 (segment (start 153.5408 81.6336) (end 153.5408 83.0436) (width 0.25) (layer "F.Cu") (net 12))
 (segment (start 153.908402 83.411202) (end 154.991297 83.411202) (width 0.25) (layer "F.Cu") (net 12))
 (segment (start 154.991297 83.411202) (end 157.1984 85.618305) (width 0.25) (layer "F.Cu") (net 12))
 (segment (start 157.1984 85.618305) (end 157.1984 85.988604) (width 0.25) (layer "F.Cu") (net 12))
 (segment (start 152.6772 80.77) (end 153.5408 81.6336) (width 0.25) (layer "F.Cu") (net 12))
 (segment (start 153.5408 83.0436) (end 153.908402 83.411202) (width 0.25) (layer "F.Cu") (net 12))
 (segment (start 157.1984 85.988604) (end 157.2 85.990204) (width 0.25) (layer "F.Cu") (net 12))
 (segment (start 157.2 85.990204) (end 157.2 102.98) (width 0.25) (layer "F.Cu") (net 12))
 (segment (start 155.35 108.39) (end 155.6136 108.39) (width 0.25) (layer "F.Cu") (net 4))
 (segment (start 147.6632 82.3352) (end 147.648 82.32) (width 0.25) (layer "F.Cu") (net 4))
 (segment (start 147.6632 84.1886) (end 147.6632 82.3352) (width 0.25) (layer "F.Cu") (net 4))
 (segment (start 147.6632 84.1886) (end 147.3584 84.4934) (width 0.25) (layer "F.Cu") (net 4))
 (segment (start 144.65 85.051) (end 144.65 96.82) (width 0.25) (layer "F.Cu") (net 4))
 (segment (start 147.3584 84.4934) (end 145.2076 84.4934) (width 0.25) (layer "F.Cu") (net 4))
 (segment (start 145.2076 84.4934) (end 144.65 85.051) (width 0.25) (layer "F.Cu") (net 4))
 (segment (start 155.6644 108.39) (end 155.35 108.39) (width 0.25) (layer "F.Cu") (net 4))
 (via (at 147.6632 84.1886) (size 0.8) (drill 0.4) (layers "F.Cu" "B.Cu") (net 4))
 (segment (start 156.2332 107.5164) (end 156.2236 107.5164) (width 0.25) (layer "B.Cu") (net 4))
 (segment (start 156.75 106.9996) (end 156.2332 107.5164) (width 0.25) (layer "B.Cu") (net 4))
 (segment (start 147.6632 84.1886) (end 148.4272 83.4246) (width 0.25) (layer "B.Cu") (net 4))
 (segment (start 148.4272 83.4246) (end 154.227996 83.4246) (width 0.25) (layer "B.Cu") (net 4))
 (segment (start 156.2236 107.5164) (end 155.35 108.39) (width 0.25) (layer "B.Cu") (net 4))
 (segment (start 154.227996 83.4246) (end 156.75 85.946604) (width 0.25) (layer "B.Cu") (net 4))
 (segment (start 156.75 85.946604) (end 156.75 106.9996) (width 0.25) (layer "B.Cu") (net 4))
 (segment (start 155.6624 110.17) (end 155.35 110.17) (width 0.25) (layer "F.Cu") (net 3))
 (segment (start 156.03 82.32) (end 154.3536 82.32) (width 0.25) (layer "F.Cu") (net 3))
 (segment (start 155.35 110.17) (end 155.6116 110.17) (width 0.25) (layer "F.Cu") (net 3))
 (segment (start 156.826 84.220599) (end 156.03 83.424599) (width 0.25) (layer "F.Cu") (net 3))
 (segment (start 156.03 83.424599) (end 156.03 82.32) (width 0.25) (layer "F.Cu") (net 3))
 (via (at 156.826 84.220599) (size 0.8) (drill 0.4) (layers "F.Cu" "B.Cu") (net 3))
 (segment (start 157.2 84.594599) (end 157.2 108.32) (width 0.25) (layer "B.Cu") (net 3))
 (segment (start 156.826 84.220599) (end 157.2 84.594599) (width 0.25) (layer "B.Cu") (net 3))
 (segment (start 157.2 108.32) (end 155.35 110.17) (width 0.25) (layer "B.Cu") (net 3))
 (segment (start 153.9988 79.0406) (end 154.1868 78.8526) (width 0.25) (layer "F.Cu") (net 1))
 (segment (start 152.1476 79.0406) (end 153.9988 79.0406) (width 0.25) (layer "F.Cu") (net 1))
 (segment (start 155.35 97.71) (end 155.35 99.49) (width 0.25) (layer "F.Cu") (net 15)))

